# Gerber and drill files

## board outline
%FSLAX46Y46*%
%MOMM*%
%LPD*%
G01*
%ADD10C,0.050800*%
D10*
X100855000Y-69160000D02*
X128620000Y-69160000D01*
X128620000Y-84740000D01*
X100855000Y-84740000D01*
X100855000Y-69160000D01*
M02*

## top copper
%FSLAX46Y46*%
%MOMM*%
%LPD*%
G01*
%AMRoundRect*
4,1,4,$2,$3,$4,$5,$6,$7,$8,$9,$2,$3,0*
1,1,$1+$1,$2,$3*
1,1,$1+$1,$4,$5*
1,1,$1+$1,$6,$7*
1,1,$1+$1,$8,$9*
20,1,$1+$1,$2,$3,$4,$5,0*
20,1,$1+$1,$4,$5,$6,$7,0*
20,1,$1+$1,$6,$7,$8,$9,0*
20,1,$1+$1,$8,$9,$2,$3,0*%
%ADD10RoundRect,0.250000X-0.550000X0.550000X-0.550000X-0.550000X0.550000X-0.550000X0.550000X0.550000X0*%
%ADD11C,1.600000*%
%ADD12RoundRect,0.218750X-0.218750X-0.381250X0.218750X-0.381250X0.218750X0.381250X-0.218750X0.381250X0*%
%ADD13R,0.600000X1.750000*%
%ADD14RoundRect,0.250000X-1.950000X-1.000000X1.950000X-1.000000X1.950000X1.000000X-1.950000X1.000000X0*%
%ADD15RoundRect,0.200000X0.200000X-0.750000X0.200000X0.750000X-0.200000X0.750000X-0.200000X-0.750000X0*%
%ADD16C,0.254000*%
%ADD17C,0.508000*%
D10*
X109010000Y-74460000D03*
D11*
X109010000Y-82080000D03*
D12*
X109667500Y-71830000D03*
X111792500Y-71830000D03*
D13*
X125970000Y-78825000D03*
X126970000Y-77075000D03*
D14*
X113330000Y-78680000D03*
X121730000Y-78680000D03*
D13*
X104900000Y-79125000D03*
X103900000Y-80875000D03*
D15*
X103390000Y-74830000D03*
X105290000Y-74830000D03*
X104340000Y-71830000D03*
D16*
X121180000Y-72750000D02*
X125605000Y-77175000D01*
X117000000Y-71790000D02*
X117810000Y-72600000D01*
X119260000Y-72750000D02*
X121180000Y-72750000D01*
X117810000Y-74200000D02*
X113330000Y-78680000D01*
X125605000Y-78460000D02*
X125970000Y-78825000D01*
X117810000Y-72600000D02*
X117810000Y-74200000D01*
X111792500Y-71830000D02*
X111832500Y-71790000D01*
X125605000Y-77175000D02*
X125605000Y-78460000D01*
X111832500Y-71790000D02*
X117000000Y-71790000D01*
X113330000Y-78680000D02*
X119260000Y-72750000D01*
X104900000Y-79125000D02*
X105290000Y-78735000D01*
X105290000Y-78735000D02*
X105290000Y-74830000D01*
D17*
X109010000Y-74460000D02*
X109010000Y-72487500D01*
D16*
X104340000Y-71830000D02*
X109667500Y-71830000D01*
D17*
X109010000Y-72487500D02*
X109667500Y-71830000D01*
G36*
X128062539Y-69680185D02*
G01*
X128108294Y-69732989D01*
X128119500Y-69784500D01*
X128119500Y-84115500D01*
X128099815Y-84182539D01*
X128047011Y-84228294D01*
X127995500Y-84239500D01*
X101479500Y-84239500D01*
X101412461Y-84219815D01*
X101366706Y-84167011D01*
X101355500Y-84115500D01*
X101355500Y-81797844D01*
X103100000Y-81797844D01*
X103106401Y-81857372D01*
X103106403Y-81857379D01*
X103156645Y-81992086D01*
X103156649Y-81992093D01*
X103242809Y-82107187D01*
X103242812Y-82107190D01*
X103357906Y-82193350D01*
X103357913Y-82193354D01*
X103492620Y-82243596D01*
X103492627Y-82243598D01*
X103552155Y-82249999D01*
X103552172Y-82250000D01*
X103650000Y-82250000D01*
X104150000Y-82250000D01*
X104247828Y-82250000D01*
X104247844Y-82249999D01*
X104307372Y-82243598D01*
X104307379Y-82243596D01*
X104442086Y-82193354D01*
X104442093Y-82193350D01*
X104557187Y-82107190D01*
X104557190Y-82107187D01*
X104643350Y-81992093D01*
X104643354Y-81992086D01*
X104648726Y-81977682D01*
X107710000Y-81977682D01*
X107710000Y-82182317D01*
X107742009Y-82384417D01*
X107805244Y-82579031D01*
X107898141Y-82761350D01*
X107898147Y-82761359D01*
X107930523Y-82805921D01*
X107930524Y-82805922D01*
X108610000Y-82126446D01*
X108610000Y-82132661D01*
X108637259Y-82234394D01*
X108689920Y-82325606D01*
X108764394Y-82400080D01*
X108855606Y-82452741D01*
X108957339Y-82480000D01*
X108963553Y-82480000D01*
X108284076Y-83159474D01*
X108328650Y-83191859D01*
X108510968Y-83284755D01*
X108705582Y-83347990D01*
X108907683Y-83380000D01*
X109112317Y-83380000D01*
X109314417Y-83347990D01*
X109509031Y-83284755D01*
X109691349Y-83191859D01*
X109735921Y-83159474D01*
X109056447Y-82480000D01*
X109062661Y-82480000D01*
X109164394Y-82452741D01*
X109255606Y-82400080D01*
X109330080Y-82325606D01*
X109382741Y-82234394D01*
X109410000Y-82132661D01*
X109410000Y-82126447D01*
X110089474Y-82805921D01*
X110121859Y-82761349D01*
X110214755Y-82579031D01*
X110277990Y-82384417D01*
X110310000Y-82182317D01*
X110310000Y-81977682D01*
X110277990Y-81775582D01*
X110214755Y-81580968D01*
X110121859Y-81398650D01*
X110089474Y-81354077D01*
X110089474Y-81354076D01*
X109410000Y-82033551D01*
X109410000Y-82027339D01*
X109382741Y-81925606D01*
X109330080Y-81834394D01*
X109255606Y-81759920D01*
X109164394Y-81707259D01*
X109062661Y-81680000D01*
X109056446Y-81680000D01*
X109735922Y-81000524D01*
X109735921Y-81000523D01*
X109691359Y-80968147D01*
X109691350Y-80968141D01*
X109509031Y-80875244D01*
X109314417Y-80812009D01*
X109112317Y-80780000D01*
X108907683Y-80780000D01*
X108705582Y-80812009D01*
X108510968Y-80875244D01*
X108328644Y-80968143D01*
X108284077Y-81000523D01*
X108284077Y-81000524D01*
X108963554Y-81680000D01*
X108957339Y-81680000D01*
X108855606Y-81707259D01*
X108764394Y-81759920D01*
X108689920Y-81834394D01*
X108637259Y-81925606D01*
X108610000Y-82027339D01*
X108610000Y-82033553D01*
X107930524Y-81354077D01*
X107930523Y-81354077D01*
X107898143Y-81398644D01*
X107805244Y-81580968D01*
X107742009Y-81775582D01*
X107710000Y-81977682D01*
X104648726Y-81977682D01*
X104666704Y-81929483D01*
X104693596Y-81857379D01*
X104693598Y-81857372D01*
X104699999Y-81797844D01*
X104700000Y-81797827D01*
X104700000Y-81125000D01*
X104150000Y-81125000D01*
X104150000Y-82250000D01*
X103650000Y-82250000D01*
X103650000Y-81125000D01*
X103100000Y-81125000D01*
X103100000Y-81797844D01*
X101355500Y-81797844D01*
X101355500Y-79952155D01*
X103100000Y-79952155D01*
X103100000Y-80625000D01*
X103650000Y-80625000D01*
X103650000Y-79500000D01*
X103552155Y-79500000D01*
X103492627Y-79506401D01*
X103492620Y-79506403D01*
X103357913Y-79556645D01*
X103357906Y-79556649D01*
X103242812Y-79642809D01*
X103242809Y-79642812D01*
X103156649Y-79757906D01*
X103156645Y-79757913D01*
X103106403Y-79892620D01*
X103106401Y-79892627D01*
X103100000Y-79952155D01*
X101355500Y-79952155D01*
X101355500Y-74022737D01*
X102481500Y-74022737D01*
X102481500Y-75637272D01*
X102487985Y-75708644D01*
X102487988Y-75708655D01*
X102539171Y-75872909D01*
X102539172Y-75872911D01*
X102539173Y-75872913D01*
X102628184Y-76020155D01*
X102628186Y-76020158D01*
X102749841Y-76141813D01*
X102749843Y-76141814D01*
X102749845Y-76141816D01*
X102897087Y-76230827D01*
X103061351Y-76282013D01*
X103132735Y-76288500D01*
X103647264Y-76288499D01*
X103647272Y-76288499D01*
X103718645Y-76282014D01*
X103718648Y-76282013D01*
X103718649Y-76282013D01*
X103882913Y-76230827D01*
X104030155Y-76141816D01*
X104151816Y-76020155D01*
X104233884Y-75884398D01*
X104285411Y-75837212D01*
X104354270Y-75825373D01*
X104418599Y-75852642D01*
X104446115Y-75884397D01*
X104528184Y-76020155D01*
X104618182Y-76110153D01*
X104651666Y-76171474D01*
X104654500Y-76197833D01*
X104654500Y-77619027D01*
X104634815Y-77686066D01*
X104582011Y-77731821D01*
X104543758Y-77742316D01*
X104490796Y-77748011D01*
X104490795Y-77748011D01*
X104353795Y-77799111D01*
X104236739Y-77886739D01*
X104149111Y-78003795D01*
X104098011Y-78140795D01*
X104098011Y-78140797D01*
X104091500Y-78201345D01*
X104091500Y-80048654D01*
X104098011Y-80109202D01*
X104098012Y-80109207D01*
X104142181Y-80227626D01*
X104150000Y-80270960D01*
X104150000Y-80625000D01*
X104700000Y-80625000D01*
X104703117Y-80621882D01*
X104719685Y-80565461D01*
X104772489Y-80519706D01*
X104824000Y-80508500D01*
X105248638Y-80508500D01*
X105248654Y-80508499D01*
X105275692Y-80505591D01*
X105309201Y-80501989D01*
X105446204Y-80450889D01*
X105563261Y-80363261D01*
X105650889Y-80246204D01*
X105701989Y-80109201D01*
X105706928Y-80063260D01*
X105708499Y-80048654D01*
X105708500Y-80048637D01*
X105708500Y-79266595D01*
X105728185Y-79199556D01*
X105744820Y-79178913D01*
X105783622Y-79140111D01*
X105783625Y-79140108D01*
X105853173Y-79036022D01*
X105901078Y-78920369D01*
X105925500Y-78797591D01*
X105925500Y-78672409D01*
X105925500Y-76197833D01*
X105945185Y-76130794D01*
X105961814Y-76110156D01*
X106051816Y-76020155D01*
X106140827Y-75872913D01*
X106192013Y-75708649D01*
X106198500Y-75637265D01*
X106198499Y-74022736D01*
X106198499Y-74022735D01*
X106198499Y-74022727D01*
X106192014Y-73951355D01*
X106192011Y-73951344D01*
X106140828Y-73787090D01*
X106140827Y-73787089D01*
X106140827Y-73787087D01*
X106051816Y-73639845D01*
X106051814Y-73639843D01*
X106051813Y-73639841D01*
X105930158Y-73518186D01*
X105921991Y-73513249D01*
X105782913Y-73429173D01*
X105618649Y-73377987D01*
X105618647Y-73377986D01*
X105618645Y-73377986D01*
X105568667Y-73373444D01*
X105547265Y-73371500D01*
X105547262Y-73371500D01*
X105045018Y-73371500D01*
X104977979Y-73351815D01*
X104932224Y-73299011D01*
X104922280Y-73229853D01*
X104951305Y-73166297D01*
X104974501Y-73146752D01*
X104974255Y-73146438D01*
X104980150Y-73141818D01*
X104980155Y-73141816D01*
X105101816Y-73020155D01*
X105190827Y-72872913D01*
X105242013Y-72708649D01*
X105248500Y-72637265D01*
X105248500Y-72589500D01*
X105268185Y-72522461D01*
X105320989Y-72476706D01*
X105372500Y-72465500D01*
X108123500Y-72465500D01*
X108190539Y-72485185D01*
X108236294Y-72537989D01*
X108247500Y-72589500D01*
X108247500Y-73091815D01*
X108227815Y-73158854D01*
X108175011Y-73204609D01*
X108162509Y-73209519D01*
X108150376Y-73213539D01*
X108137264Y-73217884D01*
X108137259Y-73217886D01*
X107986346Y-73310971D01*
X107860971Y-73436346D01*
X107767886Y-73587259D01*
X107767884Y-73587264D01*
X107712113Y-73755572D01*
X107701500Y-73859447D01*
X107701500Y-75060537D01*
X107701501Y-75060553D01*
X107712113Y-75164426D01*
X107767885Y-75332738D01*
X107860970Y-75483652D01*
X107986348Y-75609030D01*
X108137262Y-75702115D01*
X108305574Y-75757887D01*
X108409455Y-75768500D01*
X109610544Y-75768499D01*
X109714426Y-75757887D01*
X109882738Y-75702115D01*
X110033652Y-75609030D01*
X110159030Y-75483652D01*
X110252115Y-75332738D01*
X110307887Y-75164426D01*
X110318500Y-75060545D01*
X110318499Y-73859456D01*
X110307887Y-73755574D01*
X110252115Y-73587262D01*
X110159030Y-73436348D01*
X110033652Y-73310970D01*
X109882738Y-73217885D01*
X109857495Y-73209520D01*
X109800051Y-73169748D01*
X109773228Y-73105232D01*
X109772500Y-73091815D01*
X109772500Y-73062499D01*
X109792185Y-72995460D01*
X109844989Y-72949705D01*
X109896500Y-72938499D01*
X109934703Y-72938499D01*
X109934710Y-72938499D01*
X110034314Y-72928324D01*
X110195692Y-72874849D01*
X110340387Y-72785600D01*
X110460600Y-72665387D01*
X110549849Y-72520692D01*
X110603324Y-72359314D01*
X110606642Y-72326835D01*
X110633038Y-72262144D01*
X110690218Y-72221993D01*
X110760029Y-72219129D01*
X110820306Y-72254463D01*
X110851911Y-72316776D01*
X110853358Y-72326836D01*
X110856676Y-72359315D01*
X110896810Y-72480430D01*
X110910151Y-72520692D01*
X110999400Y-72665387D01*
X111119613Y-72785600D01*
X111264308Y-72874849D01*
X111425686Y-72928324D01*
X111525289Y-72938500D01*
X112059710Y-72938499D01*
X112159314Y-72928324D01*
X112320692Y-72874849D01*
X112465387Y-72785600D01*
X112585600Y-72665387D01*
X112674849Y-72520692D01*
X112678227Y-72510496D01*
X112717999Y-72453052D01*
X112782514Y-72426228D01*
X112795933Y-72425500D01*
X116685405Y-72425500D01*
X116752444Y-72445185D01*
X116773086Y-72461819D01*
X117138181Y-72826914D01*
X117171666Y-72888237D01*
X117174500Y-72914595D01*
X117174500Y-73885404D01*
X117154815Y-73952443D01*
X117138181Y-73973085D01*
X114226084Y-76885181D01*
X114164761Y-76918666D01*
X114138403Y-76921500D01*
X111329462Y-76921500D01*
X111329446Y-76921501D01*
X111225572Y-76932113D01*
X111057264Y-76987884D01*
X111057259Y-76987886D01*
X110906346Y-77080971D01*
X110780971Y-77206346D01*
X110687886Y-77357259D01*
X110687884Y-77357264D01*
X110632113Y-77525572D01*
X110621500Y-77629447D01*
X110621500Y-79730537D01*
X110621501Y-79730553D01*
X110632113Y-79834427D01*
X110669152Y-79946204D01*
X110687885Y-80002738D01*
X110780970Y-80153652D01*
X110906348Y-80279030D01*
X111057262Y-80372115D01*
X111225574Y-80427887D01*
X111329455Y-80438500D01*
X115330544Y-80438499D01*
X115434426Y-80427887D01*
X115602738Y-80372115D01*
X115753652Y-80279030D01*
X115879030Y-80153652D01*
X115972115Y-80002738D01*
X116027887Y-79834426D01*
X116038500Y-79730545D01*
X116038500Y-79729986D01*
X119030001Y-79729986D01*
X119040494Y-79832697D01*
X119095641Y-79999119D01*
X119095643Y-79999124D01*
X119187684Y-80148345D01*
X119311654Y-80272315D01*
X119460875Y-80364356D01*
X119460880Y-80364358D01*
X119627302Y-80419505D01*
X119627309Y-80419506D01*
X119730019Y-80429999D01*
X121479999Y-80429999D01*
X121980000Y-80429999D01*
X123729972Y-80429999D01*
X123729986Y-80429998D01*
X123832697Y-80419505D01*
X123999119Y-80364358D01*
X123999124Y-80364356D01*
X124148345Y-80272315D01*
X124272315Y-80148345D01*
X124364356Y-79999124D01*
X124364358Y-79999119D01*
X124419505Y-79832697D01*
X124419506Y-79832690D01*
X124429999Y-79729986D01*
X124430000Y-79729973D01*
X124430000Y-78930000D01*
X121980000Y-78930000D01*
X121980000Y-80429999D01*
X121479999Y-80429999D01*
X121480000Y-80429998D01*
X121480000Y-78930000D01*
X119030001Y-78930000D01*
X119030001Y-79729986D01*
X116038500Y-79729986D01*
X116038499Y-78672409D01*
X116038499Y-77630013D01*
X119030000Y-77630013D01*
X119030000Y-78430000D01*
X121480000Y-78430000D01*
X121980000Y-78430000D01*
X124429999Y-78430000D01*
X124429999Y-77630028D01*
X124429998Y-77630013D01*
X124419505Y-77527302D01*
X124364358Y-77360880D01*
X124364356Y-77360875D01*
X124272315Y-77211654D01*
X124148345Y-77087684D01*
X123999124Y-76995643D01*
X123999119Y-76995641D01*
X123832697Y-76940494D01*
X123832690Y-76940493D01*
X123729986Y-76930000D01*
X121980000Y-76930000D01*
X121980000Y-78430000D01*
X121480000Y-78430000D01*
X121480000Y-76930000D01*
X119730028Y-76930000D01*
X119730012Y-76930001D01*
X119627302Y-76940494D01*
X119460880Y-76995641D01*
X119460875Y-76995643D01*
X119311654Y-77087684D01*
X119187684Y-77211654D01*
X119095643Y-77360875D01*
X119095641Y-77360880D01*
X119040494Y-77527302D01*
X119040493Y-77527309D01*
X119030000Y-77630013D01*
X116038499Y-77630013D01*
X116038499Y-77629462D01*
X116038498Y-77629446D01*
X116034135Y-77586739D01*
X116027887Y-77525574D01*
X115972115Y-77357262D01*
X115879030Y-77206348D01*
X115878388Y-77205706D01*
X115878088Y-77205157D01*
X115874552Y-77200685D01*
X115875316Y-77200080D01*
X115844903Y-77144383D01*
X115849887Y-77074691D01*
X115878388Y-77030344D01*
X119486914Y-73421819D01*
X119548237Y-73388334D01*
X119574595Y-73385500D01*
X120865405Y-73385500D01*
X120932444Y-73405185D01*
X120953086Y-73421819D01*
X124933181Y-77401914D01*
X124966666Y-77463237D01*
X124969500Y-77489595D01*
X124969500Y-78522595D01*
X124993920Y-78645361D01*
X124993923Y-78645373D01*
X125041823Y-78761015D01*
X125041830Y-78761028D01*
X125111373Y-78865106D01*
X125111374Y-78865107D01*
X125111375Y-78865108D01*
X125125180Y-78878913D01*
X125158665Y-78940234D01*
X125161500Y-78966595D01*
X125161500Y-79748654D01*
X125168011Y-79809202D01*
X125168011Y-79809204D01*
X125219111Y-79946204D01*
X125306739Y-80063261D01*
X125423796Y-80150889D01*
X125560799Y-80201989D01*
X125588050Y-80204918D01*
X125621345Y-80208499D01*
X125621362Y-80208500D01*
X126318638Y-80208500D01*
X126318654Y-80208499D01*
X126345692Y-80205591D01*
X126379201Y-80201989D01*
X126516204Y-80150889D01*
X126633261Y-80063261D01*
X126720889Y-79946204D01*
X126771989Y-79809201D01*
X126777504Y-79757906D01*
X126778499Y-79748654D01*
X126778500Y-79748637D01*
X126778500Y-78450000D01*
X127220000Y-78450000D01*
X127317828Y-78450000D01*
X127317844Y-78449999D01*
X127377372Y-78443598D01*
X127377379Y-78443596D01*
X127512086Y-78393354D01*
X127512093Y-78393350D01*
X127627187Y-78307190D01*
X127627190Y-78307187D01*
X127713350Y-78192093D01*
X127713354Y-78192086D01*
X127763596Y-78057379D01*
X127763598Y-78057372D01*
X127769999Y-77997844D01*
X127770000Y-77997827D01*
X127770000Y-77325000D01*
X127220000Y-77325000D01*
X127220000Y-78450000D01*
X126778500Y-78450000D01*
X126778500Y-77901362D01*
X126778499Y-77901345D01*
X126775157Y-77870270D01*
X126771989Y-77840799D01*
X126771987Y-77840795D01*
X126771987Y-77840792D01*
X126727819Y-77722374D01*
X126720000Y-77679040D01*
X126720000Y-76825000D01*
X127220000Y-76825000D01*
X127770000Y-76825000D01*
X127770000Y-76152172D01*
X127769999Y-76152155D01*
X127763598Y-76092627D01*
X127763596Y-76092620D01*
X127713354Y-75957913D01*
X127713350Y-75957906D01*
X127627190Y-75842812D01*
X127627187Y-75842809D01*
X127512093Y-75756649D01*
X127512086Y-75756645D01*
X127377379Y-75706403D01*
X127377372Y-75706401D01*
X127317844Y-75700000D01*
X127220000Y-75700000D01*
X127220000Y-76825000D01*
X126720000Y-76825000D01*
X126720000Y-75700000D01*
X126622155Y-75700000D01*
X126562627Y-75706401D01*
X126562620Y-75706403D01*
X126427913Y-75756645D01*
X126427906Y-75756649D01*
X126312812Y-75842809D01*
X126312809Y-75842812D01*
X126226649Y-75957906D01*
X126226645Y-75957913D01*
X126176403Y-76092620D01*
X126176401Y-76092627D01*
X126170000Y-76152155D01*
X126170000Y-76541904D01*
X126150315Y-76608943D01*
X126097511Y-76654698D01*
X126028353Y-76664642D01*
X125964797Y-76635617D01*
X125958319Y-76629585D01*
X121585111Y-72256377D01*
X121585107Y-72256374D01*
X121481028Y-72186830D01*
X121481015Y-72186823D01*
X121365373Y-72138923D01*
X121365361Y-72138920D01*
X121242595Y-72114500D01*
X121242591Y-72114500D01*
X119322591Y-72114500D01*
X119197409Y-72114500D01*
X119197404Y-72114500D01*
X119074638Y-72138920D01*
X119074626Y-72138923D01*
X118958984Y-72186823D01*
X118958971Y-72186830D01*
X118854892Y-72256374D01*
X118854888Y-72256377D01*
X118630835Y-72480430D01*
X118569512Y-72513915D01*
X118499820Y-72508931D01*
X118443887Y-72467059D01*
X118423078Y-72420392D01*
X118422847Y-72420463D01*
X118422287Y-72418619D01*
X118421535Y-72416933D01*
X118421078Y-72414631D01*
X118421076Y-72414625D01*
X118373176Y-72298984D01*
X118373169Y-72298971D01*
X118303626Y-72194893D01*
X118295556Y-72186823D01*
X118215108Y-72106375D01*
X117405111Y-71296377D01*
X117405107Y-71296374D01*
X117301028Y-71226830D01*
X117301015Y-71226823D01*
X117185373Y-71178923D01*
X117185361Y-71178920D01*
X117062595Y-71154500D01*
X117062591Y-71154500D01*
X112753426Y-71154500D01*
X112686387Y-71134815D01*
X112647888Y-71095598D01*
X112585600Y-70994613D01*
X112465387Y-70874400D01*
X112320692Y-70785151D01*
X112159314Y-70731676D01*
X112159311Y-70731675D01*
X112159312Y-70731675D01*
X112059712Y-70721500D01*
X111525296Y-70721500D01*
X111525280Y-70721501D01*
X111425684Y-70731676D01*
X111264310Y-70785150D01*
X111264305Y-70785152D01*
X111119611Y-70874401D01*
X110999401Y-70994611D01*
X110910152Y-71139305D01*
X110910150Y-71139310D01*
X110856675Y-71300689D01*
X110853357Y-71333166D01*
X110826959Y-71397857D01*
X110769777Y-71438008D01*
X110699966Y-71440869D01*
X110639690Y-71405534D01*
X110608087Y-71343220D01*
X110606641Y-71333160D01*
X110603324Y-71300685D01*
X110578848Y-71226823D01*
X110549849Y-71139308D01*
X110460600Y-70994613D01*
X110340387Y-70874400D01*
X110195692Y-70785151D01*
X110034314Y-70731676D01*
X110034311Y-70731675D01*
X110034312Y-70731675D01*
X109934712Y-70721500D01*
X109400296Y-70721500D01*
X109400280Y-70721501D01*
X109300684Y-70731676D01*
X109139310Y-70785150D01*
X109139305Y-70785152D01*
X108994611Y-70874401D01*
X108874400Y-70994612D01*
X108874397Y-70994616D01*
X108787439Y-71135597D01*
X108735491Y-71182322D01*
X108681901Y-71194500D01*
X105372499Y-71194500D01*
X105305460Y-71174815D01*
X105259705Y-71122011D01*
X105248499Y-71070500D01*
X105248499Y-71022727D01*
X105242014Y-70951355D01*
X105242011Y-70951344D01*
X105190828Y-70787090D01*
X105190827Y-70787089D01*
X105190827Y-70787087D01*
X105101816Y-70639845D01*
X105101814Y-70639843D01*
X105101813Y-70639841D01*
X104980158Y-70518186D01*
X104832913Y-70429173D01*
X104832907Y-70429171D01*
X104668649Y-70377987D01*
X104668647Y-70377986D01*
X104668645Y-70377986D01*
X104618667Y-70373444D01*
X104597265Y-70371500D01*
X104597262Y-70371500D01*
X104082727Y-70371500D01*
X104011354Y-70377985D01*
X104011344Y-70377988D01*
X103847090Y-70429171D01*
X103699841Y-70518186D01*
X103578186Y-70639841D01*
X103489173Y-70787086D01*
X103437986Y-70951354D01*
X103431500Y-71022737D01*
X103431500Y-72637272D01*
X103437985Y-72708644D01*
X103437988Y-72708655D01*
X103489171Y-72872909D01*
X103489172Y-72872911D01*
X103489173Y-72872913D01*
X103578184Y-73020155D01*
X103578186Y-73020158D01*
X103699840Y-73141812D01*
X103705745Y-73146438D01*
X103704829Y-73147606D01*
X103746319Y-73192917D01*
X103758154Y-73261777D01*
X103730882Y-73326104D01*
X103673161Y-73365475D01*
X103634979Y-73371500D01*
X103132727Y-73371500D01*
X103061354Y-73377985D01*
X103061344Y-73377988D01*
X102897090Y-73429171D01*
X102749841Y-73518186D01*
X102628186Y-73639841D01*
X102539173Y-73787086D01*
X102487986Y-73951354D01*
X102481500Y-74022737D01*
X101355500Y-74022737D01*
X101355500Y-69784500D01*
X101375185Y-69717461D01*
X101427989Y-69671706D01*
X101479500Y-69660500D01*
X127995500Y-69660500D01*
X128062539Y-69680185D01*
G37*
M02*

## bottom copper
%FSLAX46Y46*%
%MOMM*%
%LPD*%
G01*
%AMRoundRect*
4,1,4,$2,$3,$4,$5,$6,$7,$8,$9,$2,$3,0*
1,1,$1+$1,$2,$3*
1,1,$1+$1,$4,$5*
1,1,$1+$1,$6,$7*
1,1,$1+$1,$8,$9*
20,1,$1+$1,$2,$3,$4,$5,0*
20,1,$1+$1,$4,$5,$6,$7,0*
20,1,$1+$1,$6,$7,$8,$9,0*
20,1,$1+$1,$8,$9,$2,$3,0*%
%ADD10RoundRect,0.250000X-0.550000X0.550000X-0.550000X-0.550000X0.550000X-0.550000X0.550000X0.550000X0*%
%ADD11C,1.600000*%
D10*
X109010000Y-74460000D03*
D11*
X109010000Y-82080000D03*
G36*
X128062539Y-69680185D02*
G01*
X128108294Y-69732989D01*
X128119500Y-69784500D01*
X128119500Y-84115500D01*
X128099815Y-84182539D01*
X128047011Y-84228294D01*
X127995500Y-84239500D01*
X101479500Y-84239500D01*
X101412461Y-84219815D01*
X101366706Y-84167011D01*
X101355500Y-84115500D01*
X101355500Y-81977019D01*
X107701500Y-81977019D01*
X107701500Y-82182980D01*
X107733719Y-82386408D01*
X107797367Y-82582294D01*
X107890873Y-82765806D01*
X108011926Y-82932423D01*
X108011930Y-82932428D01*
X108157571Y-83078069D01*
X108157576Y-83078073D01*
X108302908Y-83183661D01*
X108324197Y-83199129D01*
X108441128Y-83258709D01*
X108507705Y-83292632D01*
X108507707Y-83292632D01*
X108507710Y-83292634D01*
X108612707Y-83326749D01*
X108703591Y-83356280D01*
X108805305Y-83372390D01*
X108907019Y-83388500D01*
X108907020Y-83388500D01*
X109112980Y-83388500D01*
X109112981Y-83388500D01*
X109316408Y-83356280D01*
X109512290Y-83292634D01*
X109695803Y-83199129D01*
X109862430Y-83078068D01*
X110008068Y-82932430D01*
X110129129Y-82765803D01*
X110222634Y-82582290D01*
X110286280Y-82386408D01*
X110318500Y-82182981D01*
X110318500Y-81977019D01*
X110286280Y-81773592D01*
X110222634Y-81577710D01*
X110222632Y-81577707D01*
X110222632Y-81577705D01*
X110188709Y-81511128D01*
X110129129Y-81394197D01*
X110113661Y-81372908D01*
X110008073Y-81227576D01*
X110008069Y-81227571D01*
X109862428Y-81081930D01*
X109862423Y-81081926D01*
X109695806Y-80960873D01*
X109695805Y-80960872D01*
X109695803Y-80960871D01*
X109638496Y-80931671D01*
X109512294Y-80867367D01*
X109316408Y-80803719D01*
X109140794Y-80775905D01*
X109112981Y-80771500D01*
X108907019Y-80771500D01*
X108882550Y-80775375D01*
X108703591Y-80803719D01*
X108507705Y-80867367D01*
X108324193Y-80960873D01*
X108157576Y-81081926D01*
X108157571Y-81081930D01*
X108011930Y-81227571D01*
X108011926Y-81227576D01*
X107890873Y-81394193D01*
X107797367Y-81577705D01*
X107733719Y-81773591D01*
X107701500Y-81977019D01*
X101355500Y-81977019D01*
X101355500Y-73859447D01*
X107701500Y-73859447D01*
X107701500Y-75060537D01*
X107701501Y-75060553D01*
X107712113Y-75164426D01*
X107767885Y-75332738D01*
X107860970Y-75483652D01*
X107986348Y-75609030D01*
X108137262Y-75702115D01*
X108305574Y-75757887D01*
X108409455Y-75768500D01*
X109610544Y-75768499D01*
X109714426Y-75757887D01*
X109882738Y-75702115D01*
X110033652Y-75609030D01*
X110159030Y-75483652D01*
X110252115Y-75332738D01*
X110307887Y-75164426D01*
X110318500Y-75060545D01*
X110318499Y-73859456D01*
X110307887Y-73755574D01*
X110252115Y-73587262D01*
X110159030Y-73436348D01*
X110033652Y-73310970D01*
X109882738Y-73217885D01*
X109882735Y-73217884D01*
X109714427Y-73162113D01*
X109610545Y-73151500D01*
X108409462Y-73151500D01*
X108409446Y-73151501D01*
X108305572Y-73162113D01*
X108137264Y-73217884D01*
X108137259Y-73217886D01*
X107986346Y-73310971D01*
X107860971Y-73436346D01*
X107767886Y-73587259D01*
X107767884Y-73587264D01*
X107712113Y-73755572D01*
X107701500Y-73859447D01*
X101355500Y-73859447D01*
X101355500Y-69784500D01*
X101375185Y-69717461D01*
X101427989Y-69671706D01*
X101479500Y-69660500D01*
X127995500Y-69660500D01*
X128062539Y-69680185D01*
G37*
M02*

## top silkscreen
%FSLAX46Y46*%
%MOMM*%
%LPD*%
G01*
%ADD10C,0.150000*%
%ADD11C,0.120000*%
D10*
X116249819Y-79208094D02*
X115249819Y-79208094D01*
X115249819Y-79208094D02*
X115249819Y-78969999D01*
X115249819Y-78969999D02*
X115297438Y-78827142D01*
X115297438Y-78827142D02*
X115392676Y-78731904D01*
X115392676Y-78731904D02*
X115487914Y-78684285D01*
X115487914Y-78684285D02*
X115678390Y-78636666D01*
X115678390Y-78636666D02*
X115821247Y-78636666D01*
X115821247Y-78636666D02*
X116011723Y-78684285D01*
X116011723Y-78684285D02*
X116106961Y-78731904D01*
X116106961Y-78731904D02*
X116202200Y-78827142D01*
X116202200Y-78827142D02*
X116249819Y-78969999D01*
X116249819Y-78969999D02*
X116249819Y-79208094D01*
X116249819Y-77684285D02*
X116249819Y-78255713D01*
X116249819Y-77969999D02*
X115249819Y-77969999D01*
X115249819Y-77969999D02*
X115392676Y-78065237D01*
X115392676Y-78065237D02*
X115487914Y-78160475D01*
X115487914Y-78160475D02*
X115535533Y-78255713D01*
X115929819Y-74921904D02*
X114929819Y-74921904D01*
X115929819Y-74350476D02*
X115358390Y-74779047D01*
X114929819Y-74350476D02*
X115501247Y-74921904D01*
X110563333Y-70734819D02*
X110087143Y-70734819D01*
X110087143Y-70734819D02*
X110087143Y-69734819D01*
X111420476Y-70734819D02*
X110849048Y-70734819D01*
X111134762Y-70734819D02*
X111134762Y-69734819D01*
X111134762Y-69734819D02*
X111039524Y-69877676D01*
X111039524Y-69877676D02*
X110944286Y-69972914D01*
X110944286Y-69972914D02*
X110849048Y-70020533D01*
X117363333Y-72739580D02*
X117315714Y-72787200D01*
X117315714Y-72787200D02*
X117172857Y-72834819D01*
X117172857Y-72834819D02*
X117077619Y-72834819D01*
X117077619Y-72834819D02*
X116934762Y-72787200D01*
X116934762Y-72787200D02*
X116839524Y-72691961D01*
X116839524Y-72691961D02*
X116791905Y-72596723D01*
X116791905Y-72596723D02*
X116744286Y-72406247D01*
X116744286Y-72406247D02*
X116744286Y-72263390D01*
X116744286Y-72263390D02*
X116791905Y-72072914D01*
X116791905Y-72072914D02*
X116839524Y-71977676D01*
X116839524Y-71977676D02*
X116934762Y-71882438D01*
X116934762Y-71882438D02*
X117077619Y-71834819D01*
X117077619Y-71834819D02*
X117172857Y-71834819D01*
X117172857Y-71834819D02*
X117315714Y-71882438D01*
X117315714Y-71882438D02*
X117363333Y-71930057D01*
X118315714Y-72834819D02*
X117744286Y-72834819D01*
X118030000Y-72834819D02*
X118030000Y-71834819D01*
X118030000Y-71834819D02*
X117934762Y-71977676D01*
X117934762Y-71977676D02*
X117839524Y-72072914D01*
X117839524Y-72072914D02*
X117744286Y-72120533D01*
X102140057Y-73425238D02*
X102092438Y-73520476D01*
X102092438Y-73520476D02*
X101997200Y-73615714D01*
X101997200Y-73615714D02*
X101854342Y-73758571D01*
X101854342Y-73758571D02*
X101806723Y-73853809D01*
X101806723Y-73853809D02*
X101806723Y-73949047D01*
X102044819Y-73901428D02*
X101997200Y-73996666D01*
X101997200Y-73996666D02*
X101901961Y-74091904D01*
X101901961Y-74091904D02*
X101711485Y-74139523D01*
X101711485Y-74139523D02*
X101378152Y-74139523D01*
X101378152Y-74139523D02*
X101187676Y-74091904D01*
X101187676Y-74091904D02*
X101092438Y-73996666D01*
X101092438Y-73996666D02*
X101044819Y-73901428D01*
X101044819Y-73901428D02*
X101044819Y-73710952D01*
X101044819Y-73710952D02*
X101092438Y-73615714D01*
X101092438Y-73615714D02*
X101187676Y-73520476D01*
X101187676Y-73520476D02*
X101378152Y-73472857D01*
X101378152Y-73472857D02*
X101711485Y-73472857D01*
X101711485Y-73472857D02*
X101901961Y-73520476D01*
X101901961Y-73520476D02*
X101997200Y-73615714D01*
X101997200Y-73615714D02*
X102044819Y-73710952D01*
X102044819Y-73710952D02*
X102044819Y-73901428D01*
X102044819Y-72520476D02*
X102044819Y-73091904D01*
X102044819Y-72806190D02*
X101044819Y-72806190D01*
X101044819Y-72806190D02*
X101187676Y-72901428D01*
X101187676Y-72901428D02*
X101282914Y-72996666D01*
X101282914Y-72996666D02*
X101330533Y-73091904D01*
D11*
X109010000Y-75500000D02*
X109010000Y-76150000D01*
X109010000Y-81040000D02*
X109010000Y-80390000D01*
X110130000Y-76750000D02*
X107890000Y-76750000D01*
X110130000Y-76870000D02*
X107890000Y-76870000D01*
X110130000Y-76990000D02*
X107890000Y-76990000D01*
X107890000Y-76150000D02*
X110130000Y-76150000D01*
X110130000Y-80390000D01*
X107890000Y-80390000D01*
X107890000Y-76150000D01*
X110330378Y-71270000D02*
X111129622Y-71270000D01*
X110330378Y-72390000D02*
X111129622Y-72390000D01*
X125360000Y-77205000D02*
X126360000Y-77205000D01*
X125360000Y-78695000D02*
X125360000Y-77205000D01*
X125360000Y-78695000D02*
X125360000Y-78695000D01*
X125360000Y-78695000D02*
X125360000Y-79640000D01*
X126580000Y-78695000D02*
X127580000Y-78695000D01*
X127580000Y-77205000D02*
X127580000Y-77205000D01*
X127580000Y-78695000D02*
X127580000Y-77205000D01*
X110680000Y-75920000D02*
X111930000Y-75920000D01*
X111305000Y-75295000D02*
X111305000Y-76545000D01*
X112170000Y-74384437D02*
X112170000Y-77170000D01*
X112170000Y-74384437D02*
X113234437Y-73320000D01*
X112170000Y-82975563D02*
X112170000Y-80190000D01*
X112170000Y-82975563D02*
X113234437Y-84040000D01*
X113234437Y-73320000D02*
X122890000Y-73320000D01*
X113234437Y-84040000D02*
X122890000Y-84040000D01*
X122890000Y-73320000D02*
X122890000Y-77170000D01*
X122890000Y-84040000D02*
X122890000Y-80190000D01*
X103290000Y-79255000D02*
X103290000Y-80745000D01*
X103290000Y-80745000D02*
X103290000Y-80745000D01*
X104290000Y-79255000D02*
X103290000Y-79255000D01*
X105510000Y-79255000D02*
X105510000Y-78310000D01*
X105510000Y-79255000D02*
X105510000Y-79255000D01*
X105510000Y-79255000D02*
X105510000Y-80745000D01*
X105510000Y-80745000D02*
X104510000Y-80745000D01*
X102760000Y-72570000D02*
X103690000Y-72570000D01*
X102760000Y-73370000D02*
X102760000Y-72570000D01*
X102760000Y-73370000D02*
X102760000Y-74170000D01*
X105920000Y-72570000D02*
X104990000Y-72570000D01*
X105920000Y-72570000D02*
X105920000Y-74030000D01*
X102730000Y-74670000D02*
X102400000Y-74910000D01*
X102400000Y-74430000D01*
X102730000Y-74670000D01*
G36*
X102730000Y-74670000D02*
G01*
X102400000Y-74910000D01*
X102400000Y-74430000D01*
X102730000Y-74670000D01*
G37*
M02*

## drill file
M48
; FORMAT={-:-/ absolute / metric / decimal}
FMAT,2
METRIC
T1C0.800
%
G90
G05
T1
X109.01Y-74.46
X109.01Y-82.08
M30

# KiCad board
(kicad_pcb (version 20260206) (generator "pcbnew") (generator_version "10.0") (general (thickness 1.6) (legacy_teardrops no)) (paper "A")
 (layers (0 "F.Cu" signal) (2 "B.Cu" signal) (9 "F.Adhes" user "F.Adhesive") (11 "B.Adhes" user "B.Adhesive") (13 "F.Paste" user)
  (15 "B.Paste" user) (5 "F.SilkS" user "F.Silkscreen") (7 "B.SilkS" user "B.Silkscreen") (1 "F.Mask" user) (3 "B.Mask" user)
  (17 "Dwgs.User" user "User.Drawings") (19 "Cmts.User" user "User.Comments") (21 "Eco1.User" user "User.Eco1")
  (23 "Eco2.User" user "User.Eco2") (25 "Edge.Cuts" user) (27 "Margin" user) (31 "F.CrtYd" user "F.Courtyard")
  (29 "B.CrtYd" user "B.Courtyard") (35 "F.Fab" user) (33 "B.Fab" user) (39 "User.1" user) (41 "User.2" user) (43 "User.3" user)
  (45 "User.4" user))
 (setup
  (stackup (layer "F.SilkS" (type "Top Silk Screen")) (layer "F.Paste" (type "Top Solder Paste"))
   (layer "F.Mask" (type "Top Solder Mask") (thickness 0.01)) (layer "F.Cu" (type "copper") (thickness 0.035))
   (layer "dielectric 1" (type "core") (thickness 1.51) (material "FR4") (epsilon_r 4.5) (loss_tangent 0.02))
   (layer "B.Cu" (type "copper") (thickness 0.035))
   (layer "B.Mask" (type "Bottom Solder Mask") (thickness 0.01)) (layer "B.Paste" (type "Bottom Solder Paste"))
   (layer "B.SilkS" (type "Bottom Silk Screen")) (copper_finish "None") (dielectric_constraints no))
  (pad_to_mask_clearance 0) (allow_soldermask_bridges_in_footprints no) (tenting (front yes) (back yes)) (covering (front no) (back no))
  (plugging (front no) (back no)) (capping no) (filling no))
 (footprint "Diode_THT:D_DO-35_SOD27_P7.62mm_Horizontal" (layer "F.Cu") (at 109.01 74.46 -90)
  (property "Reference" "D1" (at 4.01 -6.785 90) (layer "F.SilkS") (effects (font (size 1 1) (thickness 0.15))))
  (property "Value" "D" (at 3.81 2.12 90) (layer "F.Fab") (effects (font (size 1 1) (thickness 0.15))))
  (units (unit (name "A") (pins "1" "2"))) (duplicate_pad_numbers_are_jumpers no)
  (fp_line (start 1.04 0) (end 1.69 0) (stroke (width 0.12) (type solid)) (layer "F.SilkS"))
  (fp_line (start 6.58 0) (end 5.93 0) (stroke (width 0.12) (type solid)) (layer "F.SilkS"))
  (fp_line (start 2.29 -1.12) (end 2.29 1.12) (stroke (width 0.12) (type solid)) (layer "F.SilkS"))
  (fp_line (start 2.41 -1.12) (end 2.41 1.12) (stroke (width 0.12) (type solid)) (layer "F.SilkS"))
  (fp_line (start 2.53 -1.12) (end 2.53 1.12) (stroke (width 0.12) (type solid)) (layer "F.SilkS"))
  (fp_rect (start 1.69 -1.12) (end 5.93 1.12) (stroke (width 0.12) (type solid)) (fill no) (layer "F.SilkS"))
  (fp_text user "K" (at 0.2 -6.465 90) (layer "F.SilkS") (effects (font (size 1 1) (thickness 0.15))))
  (pad "1" thru_hole roundrect (at 0 0 270) (size 1.6 1.6) (drill 0.8) (layers "*.Cu" "*.Mask") (remove_unused_layers no)
   (roundrect_rratio 0.15625) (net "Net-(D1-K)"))
  (pad "2" thru_hole circle (at 7.62 0 270) (size 1.6 1.6) (drill 0.8) (layers "*.Cu" "*.Mask") (remove_unused_layers no) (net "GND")))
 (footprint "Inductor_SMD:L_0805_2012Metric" (layer "F.Cu") (at 110.73 71.83)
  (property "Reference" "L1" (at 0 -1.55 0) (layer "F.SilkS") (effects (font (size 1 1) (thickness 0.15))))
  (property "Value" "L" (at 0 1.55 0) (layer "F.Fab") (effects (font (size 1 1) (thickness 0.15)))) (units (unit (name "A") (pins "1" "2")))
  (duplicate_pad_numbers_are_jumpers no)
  (fp_line (start -0.399622 -0.56) (end 0.399622 -0.56) (stroke (width 0.12) (type solid)) (layer "F.SilkS"))
  (fp_line (start -0.399622 0.56) (end 0.399622 0.56) (stroke (width 0.12) (type solid)) (layer "F.SilkS"))
  (pad "1" smd roundrect (at -1.0625 0) (size 0.875 1.2) (layers "F.Cu" "F.Mask" "F.Paste") (roundrect_rratio 0.25) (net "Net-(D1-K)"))
  (pad "2" smd roundrect (at 1.0625 0) (size 0.875 1.2) (layers "F.Cu" "F.Mask" "F.Paste") (roundrect_rratio 0.25)
   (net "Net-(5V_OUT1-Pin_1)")))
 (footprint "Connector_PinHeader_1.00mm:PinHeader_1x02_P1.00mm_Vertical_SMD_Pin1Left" (layer "F.Cu") (at 126.47 77.95 90)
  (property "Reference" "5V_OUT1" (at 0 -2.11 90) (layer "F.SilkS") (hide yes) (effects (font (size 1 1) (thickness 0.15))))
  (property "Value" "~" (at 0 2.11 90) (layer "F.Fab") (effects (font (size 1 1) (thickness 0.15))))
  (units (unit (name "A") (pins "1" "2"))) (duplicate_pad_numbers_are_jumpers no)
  (fp_line (start 0.745 -1.11) (end 0.745 -0.11) (stroke (width 0.12) (type solid)) (layer "F.SilkS"))
  (fp_line (start -0.745 -1.11) (end 0.745 -1.11) (stroke (width 0.12) (type solid)) (layer "F.SilkS"))
  (fp_line (start -0.745 -1.11) (end -0.745 -1.11) (stroke (width 0.12) (type solid)) (layer "F.SilkS"))
  (fp_line (start -0.745 -1.11) (end -1.69 -1.11) (stroke (width 0.12) (type solid)) (layer "F.SilkS"))
  (fp_line (start -0.745 0.11) (end -0.745 1.11) (stroke (width 0.12) (type solid)) (layer "F.SilkS"))
  (fp_line (start 0.745 1.11) (end 0.745 1.11) (stroke (width 0.12) (type solid)) (layer "F.SilkS"))
  (fp_line (start -0.745 1.11) (end 0.745 1.11) (stroke (width 0.12) (type solid)) (layer "F.SilkS"))
  (pad "1" smd rect (at -0.875 -0.5 90) (size 1.75 0.6) (layers "F.Cu" "F.Mask" "F.Paste") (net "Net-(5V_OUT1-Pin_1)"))
  (pad "2" smd rect (at 0.875 0.5 90) (size 1.75 0.6) (layers "F.Cu" "F.Mask" "F.Paste") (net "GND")))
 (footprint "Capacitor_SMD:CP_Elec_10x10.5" (layer "F.Cu") (at 117.53 78.68)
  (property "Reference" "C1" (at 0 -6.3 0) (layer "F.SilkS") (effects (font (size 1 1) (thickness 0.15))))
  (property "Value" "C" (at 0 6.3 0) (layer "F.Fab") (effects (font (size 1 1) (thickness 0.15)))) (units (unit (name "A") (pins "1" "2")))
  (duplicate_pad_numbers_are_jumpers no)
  (fp_line (start -6.85 -2.76) (end -5.6 -2.76) (stroke (width 0.12) (type solid)) (layer "F.SilkS"))
  (fp_line (start -6.225 -3.385) (end -6.225 -2.135) (stroke (width 0.12) (type solid)) (layer "F.SilkS"))
  (fp_line (start -5.36 -4.295563) (end -5.36 -1.51) (stroke (width 0.12) (type solid)) (layer "F.SilkS"))
  (fp_line (start -5.36 -4.295563) (end -4.295563 -5.36) (stroke (width 0.12) (type solid)) (layer "F.SilkS"))
  (fp_line (start -5.36 4.295563) (end -5.36 1.51) (stroke (width 0.12) (type solid)) (layer "F.SilkS"))
  (fp_line (start -5.36 4.295563) (end -4.295563 5.36) (stroke (width 0.12) (type solid)) (layer "F.SilkS"))
  (fp_line (start -4.295563 -5.36) (end 5.36 -5.36) (stroke (width 0.12) (type solid)) (layer "F.SilkS"))
  (fp_line (start -4.295563 5.36) (end 5.36 5.36) (stroke (width 0.12) (type solid)) (layer "F.SilkS"))
  (fp_line (start 5.36 -5.36) (end 5.36 -1.51) (stroke (width 0.12) (type solid)) (layer "F.SilkS"))
  (fp_line (start 5.36 5.36) (end 5.36 1.51) (stroke (width 0.12) (type solid)) (layer "F.SilkS"))
  (pad "1" smd roundrect (at -4.2 0) (size 4.4 2.5) (layers "F.Cu" "F.Mask" "F.Paste") (roundrect_rratio 0.1) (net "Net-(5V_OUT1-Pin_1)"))
  (pad "2" smd roundrect (at 4.2 0) (size 4.4 2.5) (layers "F.Cu" "F.Mask" "F.Paste") (roundrect_rratio 0.1) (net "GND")))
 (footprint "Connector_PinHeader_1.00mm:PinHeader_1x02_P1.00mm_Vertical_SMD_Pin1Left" (layer "F.Cu") (at 104.4 80 -90)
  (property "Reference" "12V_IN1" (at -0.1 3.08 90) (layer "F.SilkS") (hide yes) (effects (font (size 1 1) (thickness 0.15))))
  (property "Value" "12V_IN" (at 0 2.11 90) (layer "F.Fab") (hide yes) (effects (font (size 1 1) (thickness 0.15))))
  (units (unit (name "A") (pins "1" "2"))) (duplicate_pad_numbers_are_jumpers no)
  (fp_line (start -0.745 1.11) (end 0.745 1.11) (stroke (width 0.12) (type solid)) (layer "F.SilkS"))
  (fp_line (start 0.745 1.11) (end 0.745 1.11) (stroke (width 0.12) (type solid)) (layer "F.SilkS"))
  (fp_line (start -0.745 0.11) (end -0.745 1.11) (stroke (width 0.12) (type solid)) (layer "F.SilkS"))
  (fp_line (start -0.745 -1.11) (end -1.69 -1.11) (stroke (width 0.12) (type solid)) (layer "F.SilkS"))
  (fp_line (start -0.745 -1.11) (end -0.745 -1.11) (stroke (width 0.12) (type solid)) (layer "F.SilkS"))
  (fp_line (start -0.745 -1.11) (end 0.745 -1.11) (stroke (width 0.12) (type solid)) (layer "F.SilkS"))
  (fp_line (start 0.745 -1.11) (end 0.745 -0.11) (stroke (width 0.12) (type solid)) (layer "F.SilkS"))
  (pad "1" smd rect (at -0.875 -0.5 270) (size 1.75 0.6) (layers "F.Cu" "F.Mask" "F.Paste") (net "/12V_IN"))
  (pad "2" smd rect (at 0.875 0.5 270) (size 1.75 0.6) (layers "F.Cu" "F.Mask" "F.Paste") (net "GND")))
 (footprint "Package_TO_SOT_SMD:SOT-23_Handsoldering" (layer "F.Cu") (at 104.34 73.33 90)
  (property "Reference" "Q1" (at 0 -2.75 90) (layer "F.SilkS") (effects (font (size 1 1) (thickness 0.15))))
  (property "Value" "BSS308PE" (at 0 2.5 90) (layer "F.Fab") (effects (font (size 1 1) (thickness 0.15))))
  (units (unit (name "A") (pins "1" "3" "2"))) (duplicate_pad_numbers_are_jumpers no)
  (fp_line (start 0.76 -1.58) (end 0.76 -0.65) (stroke (width 0.12) (type solid)) (layer "F.SilkS"))
  (fp_line (start -0.04 -1.58) (end 0.76 -1.58) (stroke (width 0.12) (type solid)) (layer "F.SilkS"))
  (fp_line (start -0.04 -1.58) (end -0.84 -1.58) (stroke (width 0.12) (type solid)) (layer "F.SilkS"))
  (fp_line (start 0.76 1.58) (end 0.76 0.65) (stroke (width 0.12) (type solid)) (layer "F.SilkS"))
  (fp_line (start 0.76 1.58) (end -0.7 1.58) (stroke (width 0.12) (type solid)) (layer "F.SilkS"))
  (fp_poly
   (pts (xy -1.34 -1.61) (xy -1.58 -1.94) (xy -1.1 -1.94) (xy -1.34 -1.61)) (stroke (width 0.12) (type solid)) (fill yes) (layer "F.SilkS"))
  (pad "1" smd roundrect (at -1.5 -0.95 90) (size 1.9 0.8) (layers "F.Cu" "F.Mask" "F.Paste") (roundrect_rratio 0.25)
   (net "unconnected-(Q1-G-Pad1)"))
  (pad "2" smd roundrect (at -1.5 0.95 90) (size 1.9 0.8) (layers "F.Cu" "F.Mask" "F.Paste") (roundrect_rratio 0.25) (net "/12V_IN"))
  (pad "3" smd roundrect (at 1.5 0 90) (size 1.9 0.8) (layers "F.Cu" "F.Mask" "F.Paste") (roundrect_rratio 0.25) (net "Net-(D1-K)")))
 (gr_rect (start 100.855 69.16) (end 128.62 84.74) (stroke (width 0.0508) (type default)) (fill no) (layer "Edge.Cuts"))
 (segment (start 121.18 72.75) (end 125.605 77.175) (width 0.254) (layer "F.Cu") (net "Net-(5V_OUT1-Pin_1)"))
 (segment (start 117 71.79) (end 117.81 72.6) (width 0.254) (layer "F.Cu") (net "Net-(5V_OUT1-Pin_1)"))
 (segment (start 119.26 72.75) (end 121.18 72.75) (width 0.254) (layer "F.Cu") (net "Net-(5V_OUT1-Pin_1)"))
 (segment (start 117.81 74.2) (end 113.33 78.68) (width 0.254) (layer "F.Cu") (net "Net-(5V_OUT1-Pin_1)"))
 (segment (start 125.605 78.46) (end 125.97 78.825) (width 0.254) (layer "F.Cu") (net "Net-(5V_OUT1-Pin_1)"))
 (segment (start 117.81 72.6) (end 117.81 74.2) (width 0.254) (layer "F.Cu") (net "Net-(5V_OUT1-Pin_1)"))
 (segment (start 111.7925 71.83) (end 111.8325 71.79) (width 0.254) (layer "F.Cu") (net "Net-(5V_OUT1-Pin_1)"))
 (segment (start 125.605 77.175) (end 125.605 78.46) (width 0.254) (layer "F.Cu") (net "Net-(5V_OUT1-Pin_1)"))
 (segment (start 111.8325 71.79) (end 117 71.79) (width 0.254) (layer "F.Cu") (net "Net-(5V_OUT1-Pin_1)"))
 (segment (start 113.33 78.68) (end 119.26 72.75) (width 0.254) (layer "F.Cu") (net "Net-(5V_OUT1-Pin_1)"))
 (segment (start 104.9 79.125) (end 105.29 78.735) (width 0.254) (layer "F.Cu") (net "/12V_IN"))
 (segment (start 105.29 78.735) (end 105.29 74.83) (width 0.254) (layer "F.Cu") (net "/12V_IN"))
 (segment (start 109.01 74.46) (end 109.01 72.4875) (width 0.508) (layer "F.Cu") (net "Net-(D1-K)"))
 (segment (start 104.34 71.83) (end 109.6675 71.83) (width 0.254) (layer "F.Cu") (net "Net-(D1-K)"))
 (segment (start 109.01 72.4875) (end 109.6675 71.83) (width 0.508) (layer "F.Cu") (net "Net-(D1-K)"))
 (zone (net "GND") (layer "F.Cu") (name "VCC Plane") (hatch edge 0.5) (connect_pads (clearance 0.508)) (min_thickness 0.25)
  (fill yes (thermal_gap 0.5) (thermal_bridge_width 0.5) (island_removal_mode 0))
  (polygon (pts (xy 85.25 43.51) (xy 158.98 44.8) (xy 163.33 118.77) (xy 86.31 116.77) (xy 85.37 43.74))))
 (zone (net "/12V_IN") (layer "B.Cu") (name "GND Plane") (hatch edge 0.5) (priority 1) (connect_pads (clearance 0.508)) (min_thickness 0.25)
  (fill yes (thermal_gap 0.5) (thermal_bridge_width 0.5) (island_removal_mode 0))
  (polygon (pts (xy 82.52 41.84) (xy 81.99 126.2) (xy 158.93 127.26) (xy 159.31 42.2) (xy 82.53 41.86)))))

